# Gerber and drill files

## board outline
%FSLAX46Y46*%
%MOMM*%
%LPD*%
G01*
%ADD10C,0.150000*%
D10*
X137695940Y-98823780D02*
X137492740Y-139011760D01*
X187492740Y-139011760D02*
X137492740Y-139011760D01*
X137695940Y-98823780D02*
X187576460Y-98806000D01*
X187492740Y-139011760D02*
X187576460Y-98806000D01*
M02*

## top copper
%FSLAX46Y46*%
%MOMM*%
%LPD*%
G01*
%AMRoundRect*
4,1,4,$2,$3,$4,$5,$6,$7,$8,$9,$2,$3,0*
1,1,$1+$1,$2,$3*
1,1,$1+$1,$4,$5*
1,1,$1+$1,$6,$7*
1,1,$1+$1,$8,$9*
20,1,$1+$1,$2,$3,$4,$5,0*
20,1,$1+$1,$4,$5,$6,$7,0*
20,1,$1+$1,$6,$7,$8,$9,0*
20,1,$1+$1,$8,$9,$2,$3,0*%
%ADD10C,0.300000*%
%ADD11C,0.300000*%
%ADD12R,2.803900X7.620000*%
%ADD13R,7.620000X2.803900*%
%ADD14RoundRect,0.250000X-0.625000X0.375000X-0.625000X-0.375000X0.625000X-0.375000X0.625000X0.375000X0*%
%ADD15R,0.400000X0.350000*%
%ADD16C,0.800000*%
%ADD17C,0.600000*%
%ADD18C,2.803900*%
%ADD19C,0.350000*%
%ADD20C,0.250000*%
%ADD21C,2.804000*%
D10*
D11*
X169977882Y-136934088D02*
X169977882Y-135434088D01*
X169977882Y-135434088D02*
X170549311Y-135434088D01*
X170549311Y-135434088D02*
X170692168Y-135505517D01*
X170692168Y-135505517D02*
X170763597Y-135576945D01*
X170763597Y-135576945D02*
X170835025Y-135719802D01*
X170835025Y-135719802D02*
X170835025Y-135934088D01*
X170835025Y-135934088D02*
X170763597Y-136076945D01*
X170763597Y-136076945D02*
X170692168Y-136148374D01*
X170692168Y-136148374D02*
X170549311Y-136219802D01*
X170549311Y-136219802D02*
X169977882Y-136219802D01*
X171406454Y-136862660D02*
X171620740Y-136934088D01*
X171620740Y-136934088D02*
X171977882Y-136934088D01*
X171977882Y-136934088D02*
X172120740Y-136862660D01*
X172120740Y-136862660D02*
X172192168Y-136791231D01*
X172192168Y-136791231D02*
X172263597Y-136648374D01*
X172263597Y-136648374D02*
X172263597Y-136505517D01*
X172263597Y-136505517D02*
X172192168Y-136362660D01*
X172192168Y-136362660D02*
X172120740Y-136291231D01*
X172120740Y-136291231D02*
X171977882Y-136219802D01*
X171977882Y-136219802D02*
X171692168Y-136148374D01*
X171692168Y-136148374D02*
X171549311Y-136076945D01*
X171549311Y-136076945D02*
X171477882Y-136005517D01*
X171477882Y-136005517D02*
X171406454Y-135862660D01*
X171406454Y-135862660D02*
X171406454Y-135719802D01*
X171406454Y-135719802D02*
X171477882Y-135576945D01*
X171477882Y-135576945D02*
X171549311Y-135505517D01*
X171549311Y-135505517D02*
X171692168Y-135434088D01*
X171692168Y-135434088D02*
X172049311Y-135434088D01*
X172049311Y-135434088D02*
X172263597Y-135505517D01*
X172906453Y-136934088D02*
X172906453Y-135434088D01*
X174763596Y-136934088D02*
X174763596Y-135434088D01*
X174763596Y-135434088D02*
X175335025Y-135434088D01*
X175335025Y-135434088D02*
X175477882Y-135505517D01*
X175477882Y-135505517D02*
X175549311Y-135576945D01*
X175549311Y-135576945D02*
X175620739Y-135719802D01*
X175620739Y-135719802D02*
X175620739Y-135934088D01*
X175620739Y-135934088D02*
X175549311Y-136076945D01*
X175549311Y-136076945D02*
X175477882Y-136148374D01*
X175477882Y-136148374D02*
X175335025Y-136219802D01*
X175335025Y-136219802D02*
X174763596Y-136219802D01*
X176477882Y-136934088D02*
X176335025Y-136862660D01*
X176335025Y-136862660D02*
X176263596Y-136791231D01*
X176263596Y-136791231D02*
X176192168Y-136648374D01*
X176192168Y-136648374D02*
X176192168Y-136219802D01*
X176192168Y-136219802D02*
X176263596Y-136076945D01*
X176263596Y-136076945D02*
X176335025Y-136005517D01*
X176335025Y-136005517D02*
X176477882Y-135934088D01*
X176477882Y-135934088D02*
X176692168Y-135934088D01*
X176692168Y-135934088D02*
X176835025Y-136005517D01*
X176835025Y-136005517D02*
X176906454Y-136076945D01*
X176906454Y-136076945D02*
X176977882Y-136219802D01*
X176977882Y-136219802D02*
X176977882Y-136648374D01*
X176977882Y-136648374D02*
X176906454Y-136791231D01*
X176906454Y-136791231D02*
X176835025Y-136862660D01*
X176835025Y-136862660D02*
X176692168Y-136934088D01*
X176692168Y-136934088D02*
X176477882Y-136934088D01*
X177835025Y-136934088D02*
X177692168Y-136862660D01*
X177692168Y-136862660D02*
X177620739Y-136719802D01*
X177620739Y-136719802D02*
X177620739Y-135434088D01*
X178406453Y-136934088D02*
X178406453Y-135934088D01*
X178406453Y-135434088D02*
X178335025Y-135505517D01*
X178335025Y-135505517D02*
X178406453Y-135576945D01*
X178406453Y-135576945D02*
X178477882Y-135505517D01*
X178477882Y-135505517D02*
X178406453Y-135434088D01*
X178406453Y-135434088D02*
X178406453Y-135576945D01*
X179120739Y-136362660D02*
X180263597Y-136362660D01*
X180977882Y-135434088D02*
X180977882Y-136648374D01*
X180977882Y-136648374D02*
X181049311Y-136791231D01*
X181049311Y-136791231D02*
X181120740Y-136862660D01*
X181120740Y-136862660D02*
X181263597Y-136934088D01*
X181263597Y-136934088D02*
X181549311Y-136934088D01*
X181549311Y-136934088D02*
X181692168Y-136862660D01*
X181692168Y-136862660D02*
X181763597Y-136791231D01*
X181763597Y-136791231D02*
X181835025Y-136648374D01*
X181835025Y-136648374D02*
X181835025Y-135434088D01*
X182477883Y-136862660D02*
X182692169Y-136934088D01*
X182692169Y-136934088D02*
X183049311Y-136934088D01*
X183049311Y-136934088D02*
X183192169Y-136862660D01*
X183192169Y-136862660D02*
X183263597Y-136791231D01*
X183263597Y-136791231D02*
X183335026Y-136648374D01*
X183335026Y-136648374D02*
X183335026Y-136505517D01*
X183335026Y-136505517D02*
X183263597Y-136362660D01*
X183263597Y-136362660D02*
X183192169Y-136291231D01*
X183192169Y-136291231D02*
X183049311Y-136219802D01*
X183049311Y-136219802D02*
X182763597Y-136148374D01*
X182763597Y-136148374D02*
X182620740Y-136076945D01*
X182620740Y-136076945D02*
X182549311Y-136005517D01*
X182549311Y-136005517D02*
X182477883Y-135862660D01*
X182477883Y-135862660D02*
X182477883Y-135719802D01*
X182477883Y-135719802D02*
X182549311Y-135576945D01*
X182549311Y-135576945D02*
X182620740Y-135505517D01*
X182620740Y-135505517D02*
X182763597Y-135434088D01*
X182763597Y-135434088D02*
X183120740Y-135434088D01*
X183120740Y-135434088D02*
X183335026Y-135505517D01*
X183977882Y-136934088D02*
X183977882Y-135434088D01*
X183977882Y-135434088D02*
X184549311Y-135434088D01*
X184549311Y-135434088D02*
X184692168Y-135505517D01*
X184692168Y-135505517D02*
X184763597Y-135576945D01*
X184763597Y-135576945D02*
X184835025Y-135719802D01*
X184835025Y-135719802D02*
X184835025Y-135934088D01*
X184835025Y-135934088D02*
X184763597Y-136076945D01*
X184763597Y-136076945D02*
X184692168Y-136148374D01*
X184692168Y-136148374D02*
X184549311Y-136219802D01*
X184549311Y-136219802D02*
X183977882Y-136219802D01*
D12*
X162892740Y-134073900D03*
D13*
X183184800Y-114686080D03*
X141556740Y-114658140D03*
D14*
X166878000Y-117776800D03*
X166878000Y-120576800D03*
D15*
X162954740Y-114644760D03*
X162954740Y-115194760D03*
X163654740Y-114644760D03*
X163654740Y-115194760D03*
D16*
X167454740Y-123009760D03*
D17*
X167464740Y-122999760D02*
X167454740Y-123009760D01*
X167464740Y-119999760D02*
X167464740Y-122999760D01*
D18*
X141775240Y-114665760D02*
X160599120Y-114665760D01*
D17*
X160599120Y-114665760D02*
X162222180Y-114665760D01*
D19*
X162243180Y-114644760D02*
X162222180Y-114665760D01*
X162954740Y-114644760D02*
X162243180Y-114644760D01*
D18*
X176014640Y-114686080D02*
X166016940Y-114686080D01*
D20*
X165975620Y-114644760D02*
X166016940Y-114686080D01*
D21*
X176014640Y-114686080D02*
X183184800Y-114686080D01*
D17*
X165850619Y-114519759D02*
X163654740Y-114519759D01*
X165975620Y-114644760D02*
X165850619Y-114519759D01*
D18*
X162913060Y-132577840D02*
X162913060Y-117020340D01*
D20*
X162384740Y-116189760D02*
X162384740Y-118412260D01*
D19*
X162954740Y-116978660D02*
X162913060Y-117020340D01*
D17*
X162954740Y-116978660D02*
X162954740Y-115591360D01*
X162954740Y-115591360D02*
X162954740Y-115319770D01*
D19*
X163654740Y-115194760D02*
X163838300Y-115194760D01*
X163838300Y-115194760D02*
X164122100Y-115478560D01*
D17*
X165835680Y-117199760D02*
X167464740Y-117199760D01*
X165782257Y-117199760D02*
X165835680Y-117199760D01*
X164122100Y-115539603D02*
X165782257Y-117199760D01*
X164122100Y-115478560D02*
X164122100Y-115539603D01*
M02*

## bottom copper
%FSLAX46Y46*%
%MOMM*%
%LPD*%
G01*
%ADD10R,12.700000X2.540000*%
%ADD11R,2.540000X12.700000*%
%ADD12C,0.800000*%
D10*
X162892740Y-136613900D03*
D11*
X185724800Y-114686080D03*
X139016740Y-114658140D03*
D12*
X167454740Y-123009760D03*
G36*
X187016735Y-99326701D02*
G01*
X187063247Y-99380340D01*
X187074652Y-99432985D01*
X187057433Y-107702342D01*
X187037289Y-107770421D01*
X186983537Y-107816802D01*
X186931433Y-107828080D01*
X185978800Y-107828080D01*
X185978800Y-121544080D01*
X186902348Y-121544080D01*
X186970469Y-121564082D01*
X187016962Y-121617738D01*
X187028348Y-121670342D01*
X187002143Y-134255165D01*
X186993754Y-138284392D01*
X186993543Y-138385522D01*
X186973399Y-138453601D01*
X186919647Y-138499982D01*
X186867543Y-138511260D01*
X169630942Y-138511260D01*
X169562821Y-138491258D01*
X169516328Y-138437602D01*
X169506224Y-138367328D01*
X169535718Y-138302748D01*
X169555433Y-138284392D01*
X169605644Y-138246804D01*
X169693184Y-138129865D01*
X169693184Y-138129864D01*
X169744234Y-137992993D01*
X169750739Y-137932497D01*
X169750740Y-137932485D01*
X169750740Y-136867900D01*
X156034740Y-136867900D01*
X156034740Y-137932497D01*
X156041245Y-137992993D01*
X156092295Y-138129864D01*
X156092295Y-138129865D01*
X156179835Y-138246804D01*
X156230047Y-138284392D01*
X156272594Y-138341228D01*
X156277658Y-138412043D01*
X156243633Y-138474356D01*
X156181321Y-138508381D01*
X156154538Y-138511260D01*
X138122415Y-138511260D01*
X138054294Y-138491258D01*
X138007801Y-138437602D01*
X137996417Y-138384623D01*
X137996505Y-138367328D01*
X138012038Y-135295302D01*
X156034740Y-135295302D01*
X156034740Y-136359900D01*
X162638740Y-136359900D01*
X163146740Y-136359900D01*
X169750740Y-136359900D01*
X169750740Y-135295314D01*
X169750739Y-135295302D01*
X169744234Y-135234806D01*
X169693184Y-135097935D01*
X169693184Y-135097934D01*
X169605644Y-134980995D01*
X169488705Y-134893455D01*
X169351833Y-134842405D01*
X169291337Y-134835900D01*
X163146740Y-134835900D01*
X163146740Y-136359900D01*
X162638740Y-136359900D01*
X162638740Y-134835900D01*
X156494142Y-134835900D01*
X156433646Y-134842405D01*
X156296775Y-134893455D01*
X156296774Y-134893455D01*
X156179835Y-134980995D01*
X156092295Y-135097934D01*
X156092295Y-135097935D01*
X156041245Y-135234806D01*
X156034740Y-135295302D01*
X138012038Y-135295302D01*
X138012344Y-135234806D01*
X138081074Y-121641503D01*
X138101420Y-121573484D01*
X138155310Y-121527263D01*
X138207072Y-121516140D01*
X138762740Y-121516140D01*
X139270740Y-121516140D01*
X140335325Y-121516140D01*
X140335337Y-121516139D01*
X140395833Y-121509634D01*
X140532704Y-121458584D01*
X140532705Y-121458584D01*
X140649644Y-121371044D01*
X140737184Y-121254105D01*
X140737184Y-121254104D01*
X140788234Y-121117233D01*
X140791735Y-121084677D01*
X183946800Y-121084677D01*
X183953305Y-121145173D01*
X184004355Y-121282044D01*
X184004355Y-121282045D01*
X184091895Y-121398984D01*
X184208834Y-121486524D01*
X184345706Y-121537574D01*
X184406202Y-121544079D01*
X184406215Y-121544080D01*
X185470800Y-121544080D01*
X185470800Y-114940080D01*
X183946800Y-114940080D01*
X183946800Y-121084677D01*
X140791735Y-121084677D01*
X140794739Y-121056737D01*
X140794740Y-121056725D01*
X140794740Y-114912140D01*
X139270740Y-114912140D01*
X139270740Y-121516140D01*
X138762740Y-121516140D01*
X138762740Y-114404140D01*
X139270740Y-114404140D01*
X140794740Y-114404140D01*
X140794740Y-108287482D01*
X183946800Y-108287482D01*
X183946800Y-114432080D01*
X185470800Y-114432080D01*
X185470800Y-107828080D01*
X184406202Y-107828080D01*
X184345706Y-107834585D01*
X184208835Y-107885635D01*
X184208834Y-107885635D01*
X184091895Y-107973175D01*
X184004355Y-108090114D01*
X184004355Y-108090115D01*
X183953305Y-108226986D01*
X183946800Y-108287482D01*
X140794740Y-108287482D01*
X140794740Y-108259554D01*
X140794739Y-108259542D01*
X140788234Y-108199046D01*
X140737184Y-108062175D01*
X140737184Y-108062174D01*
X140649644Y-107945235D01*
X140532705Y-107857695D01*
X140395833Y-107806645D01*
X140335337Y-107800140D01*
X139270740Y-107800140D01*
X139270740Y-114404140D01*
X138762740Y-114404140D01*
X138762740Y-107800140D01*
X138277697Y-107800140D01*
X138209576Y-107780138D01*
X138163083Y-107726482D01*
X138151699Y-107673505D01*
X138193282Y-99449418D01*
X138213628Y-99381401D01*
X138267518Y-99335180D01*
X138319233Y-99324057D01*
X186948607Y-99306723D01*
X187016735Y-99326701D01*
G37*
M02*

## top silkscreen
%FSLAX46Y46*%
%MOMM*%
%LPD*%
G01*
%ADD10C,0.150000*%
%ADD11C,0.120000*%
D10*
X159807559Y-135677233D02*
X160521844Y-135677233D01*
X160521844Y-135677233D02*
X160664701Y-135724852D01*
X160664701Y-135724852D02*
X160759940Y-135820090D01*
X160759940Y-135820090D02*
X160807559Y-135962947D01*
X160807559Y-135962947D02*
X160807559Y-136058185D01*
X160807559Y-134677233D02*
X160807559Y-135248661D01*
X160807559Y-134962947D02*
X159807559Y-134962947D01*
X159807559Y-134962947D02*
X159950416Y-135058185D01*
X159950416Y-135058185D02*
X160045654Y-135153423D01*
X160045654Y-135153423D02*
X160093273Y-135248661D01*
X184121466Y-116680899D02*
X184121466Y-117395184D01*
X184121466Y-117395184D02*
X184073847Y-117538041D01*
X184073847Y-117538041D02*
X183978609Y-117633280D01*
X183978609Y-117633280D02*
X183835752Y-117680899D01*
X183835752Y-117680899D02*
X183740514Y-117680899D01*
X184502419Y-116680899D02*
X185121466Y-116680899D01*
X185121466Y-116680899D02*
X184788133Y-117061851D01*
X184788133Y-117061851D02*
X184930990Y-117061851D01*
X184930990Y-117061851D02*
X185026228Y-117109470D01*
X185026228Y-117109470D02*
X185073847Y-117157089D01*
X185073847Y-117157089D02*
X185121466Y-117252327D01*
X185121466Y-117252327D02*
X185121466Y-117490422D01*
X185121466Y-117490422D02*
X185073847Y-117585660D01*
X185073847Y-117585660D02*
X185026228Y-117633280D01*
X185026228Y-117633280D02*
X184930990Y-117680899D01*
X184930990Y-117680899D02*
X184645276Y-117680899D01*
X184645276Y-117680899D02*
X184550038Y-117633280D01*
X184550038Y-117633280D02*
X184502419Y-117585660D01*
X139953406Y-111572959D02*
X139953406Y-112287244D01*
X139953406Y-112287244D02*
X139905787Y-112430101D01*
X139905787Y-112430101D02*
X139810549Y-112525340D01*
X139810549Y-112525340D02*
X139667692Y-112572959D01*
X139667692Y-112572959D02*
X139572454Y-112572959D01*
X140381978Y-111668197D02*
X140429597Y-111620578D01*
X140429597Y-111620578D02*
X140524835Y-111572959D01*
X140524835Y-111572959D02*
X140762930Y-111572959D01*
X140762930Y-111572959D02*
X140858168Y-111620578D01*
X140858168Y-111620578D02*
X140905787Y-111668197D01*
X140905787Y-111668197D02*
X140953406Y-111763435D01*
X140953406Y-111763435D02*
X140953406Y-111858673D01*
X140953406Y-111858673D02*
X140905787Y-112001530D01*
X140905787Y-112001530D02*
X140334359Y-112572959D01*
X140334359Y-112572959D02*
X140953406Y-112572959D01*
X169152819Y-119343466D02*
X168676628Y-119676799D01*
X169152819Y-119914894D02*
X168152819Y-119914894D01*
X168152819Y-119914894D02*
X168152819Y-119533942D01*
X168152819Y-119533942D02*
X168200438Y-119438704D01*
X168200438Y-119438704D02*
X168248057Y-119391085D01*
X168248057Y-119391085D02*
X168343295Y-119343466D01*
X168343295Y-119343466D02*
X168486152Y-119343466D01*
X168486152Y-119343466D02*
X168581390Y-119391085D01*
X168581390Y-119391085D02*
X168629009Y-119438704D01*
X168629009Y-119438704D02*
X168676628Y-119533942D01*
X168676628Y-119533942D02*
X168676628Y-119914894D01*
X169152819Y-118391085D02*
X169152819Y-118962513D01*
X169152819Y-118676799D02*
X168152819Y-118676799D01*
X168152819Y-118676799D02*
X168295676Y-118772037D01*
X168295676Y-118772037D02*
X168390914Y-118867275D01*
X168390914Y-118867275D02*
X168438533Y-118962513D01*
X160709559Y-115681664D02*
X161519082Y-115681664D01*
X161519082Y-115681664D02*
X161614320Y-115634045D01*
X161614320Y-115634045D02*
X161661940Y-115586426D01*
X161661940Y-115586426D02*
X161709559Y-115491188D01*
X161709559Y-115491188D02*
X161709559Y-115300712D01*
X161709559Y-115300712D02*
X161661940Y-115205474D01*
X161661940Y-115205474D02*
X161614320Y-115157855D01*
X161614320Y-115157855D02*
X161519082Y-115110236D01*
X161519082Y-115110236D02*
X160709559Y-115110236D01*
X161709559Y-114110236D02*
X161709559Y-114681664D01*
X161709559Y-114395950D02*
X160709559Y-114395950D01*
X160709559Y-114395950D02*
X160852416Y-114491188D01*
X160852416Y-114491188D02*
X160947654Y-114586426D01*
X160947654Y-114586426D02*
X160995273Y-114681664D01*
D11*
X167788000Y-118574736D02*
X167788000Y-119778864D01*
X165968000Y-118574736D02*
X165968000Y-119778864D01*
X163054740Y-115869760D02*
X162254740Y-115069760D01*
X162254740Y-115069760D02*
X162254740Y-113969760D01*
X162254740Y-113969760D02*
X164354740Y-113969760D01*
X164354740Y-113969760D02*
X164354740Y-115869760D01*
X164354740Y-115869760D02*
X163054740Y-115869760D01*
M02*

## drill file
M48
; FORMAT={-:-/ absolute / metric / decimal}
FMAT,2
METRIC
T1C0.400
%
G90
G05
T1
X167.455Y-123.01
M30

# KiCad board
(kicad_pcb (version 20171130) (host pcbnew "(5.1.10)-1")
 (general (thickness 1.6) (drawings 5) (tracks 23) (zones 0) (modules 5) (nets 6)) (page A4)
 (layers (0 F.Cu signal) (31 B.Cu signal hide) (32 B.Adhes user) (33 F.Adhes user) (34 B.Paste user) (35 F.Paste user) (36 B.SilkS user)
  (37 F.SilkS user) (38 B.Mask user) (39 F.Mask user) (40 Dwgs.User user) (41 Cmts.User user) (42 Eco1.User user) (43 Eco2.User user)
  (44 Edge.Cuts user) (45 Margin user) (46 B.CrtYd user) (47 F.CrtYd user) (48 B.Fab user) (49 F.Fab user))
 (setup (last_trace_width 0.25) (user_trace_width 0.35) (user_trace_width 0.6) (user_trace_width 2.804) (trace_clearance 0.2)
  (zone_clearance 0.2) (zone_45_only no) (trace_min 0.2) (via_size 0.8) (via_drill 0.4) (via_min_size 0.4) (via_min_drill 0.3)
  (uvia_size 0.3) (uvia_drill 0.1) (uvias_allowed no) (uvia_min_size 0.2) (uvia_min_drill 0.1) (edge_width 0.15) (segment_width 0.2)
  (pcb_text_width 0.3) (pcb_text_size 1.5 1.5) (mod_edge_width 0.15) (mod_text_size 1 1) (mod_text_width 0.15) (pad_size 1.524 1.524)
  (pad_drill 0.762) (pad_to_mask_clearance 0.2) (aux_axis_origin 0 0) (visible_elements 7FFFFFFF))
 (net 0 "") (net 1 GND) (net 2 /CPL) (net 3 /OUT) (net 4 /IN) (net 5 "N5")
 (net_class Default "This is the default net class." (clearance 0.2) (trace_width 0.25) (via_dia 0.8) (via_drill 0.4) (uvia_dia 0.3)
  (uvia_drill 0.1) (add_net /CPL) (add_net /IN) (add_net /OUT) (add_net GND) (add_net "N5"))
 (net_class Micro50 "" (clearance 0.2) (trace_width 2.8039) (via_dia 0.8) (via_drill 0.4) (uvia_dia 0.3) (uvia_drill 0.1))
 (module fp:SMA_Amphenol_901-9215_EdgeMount (layer F.Cu) (at 162.89274 132.8039 270)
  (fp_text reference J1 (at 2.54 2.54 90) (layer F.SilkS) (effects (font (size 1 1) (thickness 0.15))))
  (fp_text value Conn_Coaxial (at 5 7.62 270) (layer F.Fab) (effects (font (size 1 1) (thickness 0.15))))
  (pad 2 smd rect (at 3.81 0 90) (size 2.54 12.7) (layers B.Cu B.Paste B.Mask) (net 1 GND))
  (pad 1 smd rect (at 1.27 0) (size 2.8039 7.62) (layers F.Cu F.Paste F.Mask) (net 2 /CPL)))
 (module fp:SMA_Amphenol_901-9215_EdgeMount (layer F.Cu) (at 181.9148 114.68608)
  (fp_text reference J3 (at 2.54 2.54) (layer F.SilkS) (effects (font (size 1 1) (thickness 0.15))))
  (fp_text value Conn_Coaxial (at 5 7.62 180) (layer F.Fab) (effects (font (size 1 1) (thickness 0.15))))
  (pad 1 smd rect (at 1.27 0 90) (size 2.8039 7.62) (layers F.Cu F.Paste F.Mask) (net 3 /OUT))
  (pad 2 smd rect (at 3.81 0 180) (size 2.54 12.7) (layers B.Cu B.Paste B.Mask) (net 1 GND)))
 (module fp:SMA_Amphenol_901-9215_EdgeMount (layer F.Cu) (at 142.82674 114.65814 180)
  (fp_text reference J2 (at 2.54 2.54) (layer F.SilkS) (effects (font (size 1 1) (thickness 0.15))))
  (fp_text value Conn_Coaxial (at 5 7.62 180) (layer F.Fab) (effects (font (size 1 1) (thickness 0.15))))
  (pad 2 smd rect (at 3.81 0) (size 2.54 12.7) (layers B.Cu B.Paste B.Mask) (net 1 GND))
  (pad 1 smd rect (at 1.27 0 270) (size 2.8039 7.62) (layers F.Cu F.Paste F.Mask) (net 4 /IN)))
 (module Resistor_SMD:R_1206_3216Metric (layer F.Cu) (at 166.878 119.1768 270)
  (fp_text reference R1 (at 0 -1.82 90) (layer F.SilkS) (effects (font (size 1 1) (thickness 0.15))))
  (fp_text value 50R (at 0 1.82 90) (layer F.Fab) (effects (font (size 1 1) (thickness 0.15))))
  (fp_line (start -0.602064 -0.91) (end 0.602064 -0.91) (layer F.SilkS) (width 0.12))
  (fp_line (start -0.602064 0.91) (end 0.602064 0.91) (layer F.SilkS) (width 0.12))
  (pad 1 smd roundrect (at -1.4 0 270) (size 1.25 1.75) (layers F.Cu F.Paste F.Mask) (roundrect_rratio 0.2) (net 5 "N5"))
  (pad 2 smd roundrect (at 1.4 0 270) (size 1.25 1.75) (layers F.Cu F.Paste F.Mask) (roundrect_rratio 0.2) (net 1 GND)))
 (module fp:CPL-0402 (layer F.Cu) (at 163.30474 114.91976)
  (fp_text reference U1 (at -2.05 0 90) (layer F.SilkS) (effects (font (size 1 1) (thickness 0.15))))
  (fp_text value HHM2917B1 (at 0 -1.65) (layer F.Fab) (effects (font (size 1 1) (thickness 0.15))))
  (fp_line (start -0.25 0.95) (end -1.05 0.15) (layer F.SilkS) (width 0.12))
  (fp_line (start -1.05 0.15) (end -1.05 -0.95) (layer F.SilkS) (width 0.12))
  (fp_line (start -1.05 -0.95) (end 1.05 -0.95) (layer F.SilkS) (width 0.12))
  (fp_line (start 1.05 -0.95) (end 1.05 0.95) (layer F.SilkS) (width 0.12))
  (fp_line (start 1.05 0.95) (end -0.25 0.95) (layer F.SilkS) (width 0.12))
  (pad 4 smd rect (at -0.35 -0.275) (size 0.4 0.35) (layers F.Cu F.Paste F.Mask) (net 4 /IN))
  (pad 1 smd rect (at -0.35 0.275) (size 0.4 0.35) (layers F.Cu F.Paste F.Mask) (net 2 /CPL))
  (pad 3 smd rect (at 0.35 -0.275) (size 0.4 0.35) (layers F.Cu F.Paste F.Mask) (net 3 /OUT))
  (pad 2 smd rect (at 0.35 0.275) (size 0.4 0.35) (layers F.Cu F.Paste F.Mask) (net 5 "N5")))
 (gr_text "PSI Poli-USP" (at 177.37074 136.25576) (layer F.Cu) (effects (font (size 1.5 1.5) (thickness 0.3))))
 (gr_line (start 137.69594 98.82378) (end 137.49274 139.01176) (layer Edge.Cuts) (width 0.15))
 (gr_line (start 187.49274 139.01176) (end 137.49274 139.01176) (layer Edge.Cuts) (width 0.15))
 (gr_line (start 137.69594 98.82378) (end 187.57646 98.806) (layer Edge.Cuts) (width 0.15))
 (gr_line (start 187.49274 139.01176) (end 187.57646 98.806) (layer Edge.Cuts) (width 0.15))
 (via (at 167.45474 123.00976) (size 0.8) (drill 0.4) (layers F.Cu B.Cu) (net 1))
 (segment (start 167.46474 122.99976) (end 167.45474 123.00976) (width 0.6) (layer F.Cu) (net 1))
 (segment (start 167.46474 119.99976) (end 167.46474 122.99976) (width 0.6) (layer F.Cu) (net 1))
 (segment (start 141.77524 114.66576) (end 160.59912 114.66576) (width 2.8039) (layer F.Cu) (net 4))
 (segment (start 160.59912 114.66576) (end 162.22218 114.66576) (width 0.6) (layer F.Cu) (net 4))
 (segment (start 162.24318 114.64476) (end 162.22218 114.66576) (width 0.35) (layer F.Cu) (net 4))
 (segment (start 162.95474 114.64476) (end 162.24318 114.64476) (width 0.35) (layer F.Cu) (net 4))
 (segment (start 176.01464 114.68608) (end 166.01694 114.68608) (width 2.8039) (layer F.Cu) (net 3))
 (segment (start 165.97562 114.64476) (end 166.01694 114.68608) (width 0.25) (layer F.Cu) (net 3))
 (segment (start 176.01464 114.68608) (end 183.1848 114.68608) (width 2.804) (layer F.Cu) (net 3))
 (segment (start 165.850619 114.519759) (end 163.65474 114.519759) (width 0.6) (layer F.Cu) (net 3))
 (segment (start 165.97562 114.64476) (end 165.850619 114.519759) (width 0.6) (layer F.Cu) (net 3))
 (segment (start 162.91306 132.57784) (end 162.91306 117.02034) (width 2.8039) (layer F.Cu) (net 2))
 (segment (start 162.38474 116.18976) (end 162.38474 118.41226) (width 0.25) (layer F.Cu) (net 2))
 (segment (start 162.95474 116.97866) (end 162.91306 117.02034) (width 0.35) (layer F.Cu) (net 2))
 (segment (start 162.95474 116.97866) (end 162.95474 115.59136) (width 0.6) (layer F.Cu) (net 2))
 (segment (start 162.95474 115.59136) (end 162.95474 115.31977) (width 0.6) (layer F.Cu) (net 2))
 (segment (start 163.65474 115.19476) (end 163.8383 115.19476) (width 0.35) (layer F.Cu) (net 5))
 (segment (start 163.8383 115.19476) (end 164.1221 115.47856) (width 0.35) (layer F.Cu) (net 5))
 (segment (start 165.83568 117.19976) (end 167.46474 117.19976) (width 0.6) (layer F.Cu) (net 5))
 (segment (start 165.782257 117.19976) (end 165.83568 117.19976) (width 0.6) (layer F.Cu) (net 5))
 (segment (start 164.1221 115.539603) (end 165.782257 117.19976) (width 0.6) (layer F.Cu) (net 5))
 (segment (start 164.1221 115.47856) (end 164.1221 115.539603) (width 0.6) (layer F.Cu) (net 5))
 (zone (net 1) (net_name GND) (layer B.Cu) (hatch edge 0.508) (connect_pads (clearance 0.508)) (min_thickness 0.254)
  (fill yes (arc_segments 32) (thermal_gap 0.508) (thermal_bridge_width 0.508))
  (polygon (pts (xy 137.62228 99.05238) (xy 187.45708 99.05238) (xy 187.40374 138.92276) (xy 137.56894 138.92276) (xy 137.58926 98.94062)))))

